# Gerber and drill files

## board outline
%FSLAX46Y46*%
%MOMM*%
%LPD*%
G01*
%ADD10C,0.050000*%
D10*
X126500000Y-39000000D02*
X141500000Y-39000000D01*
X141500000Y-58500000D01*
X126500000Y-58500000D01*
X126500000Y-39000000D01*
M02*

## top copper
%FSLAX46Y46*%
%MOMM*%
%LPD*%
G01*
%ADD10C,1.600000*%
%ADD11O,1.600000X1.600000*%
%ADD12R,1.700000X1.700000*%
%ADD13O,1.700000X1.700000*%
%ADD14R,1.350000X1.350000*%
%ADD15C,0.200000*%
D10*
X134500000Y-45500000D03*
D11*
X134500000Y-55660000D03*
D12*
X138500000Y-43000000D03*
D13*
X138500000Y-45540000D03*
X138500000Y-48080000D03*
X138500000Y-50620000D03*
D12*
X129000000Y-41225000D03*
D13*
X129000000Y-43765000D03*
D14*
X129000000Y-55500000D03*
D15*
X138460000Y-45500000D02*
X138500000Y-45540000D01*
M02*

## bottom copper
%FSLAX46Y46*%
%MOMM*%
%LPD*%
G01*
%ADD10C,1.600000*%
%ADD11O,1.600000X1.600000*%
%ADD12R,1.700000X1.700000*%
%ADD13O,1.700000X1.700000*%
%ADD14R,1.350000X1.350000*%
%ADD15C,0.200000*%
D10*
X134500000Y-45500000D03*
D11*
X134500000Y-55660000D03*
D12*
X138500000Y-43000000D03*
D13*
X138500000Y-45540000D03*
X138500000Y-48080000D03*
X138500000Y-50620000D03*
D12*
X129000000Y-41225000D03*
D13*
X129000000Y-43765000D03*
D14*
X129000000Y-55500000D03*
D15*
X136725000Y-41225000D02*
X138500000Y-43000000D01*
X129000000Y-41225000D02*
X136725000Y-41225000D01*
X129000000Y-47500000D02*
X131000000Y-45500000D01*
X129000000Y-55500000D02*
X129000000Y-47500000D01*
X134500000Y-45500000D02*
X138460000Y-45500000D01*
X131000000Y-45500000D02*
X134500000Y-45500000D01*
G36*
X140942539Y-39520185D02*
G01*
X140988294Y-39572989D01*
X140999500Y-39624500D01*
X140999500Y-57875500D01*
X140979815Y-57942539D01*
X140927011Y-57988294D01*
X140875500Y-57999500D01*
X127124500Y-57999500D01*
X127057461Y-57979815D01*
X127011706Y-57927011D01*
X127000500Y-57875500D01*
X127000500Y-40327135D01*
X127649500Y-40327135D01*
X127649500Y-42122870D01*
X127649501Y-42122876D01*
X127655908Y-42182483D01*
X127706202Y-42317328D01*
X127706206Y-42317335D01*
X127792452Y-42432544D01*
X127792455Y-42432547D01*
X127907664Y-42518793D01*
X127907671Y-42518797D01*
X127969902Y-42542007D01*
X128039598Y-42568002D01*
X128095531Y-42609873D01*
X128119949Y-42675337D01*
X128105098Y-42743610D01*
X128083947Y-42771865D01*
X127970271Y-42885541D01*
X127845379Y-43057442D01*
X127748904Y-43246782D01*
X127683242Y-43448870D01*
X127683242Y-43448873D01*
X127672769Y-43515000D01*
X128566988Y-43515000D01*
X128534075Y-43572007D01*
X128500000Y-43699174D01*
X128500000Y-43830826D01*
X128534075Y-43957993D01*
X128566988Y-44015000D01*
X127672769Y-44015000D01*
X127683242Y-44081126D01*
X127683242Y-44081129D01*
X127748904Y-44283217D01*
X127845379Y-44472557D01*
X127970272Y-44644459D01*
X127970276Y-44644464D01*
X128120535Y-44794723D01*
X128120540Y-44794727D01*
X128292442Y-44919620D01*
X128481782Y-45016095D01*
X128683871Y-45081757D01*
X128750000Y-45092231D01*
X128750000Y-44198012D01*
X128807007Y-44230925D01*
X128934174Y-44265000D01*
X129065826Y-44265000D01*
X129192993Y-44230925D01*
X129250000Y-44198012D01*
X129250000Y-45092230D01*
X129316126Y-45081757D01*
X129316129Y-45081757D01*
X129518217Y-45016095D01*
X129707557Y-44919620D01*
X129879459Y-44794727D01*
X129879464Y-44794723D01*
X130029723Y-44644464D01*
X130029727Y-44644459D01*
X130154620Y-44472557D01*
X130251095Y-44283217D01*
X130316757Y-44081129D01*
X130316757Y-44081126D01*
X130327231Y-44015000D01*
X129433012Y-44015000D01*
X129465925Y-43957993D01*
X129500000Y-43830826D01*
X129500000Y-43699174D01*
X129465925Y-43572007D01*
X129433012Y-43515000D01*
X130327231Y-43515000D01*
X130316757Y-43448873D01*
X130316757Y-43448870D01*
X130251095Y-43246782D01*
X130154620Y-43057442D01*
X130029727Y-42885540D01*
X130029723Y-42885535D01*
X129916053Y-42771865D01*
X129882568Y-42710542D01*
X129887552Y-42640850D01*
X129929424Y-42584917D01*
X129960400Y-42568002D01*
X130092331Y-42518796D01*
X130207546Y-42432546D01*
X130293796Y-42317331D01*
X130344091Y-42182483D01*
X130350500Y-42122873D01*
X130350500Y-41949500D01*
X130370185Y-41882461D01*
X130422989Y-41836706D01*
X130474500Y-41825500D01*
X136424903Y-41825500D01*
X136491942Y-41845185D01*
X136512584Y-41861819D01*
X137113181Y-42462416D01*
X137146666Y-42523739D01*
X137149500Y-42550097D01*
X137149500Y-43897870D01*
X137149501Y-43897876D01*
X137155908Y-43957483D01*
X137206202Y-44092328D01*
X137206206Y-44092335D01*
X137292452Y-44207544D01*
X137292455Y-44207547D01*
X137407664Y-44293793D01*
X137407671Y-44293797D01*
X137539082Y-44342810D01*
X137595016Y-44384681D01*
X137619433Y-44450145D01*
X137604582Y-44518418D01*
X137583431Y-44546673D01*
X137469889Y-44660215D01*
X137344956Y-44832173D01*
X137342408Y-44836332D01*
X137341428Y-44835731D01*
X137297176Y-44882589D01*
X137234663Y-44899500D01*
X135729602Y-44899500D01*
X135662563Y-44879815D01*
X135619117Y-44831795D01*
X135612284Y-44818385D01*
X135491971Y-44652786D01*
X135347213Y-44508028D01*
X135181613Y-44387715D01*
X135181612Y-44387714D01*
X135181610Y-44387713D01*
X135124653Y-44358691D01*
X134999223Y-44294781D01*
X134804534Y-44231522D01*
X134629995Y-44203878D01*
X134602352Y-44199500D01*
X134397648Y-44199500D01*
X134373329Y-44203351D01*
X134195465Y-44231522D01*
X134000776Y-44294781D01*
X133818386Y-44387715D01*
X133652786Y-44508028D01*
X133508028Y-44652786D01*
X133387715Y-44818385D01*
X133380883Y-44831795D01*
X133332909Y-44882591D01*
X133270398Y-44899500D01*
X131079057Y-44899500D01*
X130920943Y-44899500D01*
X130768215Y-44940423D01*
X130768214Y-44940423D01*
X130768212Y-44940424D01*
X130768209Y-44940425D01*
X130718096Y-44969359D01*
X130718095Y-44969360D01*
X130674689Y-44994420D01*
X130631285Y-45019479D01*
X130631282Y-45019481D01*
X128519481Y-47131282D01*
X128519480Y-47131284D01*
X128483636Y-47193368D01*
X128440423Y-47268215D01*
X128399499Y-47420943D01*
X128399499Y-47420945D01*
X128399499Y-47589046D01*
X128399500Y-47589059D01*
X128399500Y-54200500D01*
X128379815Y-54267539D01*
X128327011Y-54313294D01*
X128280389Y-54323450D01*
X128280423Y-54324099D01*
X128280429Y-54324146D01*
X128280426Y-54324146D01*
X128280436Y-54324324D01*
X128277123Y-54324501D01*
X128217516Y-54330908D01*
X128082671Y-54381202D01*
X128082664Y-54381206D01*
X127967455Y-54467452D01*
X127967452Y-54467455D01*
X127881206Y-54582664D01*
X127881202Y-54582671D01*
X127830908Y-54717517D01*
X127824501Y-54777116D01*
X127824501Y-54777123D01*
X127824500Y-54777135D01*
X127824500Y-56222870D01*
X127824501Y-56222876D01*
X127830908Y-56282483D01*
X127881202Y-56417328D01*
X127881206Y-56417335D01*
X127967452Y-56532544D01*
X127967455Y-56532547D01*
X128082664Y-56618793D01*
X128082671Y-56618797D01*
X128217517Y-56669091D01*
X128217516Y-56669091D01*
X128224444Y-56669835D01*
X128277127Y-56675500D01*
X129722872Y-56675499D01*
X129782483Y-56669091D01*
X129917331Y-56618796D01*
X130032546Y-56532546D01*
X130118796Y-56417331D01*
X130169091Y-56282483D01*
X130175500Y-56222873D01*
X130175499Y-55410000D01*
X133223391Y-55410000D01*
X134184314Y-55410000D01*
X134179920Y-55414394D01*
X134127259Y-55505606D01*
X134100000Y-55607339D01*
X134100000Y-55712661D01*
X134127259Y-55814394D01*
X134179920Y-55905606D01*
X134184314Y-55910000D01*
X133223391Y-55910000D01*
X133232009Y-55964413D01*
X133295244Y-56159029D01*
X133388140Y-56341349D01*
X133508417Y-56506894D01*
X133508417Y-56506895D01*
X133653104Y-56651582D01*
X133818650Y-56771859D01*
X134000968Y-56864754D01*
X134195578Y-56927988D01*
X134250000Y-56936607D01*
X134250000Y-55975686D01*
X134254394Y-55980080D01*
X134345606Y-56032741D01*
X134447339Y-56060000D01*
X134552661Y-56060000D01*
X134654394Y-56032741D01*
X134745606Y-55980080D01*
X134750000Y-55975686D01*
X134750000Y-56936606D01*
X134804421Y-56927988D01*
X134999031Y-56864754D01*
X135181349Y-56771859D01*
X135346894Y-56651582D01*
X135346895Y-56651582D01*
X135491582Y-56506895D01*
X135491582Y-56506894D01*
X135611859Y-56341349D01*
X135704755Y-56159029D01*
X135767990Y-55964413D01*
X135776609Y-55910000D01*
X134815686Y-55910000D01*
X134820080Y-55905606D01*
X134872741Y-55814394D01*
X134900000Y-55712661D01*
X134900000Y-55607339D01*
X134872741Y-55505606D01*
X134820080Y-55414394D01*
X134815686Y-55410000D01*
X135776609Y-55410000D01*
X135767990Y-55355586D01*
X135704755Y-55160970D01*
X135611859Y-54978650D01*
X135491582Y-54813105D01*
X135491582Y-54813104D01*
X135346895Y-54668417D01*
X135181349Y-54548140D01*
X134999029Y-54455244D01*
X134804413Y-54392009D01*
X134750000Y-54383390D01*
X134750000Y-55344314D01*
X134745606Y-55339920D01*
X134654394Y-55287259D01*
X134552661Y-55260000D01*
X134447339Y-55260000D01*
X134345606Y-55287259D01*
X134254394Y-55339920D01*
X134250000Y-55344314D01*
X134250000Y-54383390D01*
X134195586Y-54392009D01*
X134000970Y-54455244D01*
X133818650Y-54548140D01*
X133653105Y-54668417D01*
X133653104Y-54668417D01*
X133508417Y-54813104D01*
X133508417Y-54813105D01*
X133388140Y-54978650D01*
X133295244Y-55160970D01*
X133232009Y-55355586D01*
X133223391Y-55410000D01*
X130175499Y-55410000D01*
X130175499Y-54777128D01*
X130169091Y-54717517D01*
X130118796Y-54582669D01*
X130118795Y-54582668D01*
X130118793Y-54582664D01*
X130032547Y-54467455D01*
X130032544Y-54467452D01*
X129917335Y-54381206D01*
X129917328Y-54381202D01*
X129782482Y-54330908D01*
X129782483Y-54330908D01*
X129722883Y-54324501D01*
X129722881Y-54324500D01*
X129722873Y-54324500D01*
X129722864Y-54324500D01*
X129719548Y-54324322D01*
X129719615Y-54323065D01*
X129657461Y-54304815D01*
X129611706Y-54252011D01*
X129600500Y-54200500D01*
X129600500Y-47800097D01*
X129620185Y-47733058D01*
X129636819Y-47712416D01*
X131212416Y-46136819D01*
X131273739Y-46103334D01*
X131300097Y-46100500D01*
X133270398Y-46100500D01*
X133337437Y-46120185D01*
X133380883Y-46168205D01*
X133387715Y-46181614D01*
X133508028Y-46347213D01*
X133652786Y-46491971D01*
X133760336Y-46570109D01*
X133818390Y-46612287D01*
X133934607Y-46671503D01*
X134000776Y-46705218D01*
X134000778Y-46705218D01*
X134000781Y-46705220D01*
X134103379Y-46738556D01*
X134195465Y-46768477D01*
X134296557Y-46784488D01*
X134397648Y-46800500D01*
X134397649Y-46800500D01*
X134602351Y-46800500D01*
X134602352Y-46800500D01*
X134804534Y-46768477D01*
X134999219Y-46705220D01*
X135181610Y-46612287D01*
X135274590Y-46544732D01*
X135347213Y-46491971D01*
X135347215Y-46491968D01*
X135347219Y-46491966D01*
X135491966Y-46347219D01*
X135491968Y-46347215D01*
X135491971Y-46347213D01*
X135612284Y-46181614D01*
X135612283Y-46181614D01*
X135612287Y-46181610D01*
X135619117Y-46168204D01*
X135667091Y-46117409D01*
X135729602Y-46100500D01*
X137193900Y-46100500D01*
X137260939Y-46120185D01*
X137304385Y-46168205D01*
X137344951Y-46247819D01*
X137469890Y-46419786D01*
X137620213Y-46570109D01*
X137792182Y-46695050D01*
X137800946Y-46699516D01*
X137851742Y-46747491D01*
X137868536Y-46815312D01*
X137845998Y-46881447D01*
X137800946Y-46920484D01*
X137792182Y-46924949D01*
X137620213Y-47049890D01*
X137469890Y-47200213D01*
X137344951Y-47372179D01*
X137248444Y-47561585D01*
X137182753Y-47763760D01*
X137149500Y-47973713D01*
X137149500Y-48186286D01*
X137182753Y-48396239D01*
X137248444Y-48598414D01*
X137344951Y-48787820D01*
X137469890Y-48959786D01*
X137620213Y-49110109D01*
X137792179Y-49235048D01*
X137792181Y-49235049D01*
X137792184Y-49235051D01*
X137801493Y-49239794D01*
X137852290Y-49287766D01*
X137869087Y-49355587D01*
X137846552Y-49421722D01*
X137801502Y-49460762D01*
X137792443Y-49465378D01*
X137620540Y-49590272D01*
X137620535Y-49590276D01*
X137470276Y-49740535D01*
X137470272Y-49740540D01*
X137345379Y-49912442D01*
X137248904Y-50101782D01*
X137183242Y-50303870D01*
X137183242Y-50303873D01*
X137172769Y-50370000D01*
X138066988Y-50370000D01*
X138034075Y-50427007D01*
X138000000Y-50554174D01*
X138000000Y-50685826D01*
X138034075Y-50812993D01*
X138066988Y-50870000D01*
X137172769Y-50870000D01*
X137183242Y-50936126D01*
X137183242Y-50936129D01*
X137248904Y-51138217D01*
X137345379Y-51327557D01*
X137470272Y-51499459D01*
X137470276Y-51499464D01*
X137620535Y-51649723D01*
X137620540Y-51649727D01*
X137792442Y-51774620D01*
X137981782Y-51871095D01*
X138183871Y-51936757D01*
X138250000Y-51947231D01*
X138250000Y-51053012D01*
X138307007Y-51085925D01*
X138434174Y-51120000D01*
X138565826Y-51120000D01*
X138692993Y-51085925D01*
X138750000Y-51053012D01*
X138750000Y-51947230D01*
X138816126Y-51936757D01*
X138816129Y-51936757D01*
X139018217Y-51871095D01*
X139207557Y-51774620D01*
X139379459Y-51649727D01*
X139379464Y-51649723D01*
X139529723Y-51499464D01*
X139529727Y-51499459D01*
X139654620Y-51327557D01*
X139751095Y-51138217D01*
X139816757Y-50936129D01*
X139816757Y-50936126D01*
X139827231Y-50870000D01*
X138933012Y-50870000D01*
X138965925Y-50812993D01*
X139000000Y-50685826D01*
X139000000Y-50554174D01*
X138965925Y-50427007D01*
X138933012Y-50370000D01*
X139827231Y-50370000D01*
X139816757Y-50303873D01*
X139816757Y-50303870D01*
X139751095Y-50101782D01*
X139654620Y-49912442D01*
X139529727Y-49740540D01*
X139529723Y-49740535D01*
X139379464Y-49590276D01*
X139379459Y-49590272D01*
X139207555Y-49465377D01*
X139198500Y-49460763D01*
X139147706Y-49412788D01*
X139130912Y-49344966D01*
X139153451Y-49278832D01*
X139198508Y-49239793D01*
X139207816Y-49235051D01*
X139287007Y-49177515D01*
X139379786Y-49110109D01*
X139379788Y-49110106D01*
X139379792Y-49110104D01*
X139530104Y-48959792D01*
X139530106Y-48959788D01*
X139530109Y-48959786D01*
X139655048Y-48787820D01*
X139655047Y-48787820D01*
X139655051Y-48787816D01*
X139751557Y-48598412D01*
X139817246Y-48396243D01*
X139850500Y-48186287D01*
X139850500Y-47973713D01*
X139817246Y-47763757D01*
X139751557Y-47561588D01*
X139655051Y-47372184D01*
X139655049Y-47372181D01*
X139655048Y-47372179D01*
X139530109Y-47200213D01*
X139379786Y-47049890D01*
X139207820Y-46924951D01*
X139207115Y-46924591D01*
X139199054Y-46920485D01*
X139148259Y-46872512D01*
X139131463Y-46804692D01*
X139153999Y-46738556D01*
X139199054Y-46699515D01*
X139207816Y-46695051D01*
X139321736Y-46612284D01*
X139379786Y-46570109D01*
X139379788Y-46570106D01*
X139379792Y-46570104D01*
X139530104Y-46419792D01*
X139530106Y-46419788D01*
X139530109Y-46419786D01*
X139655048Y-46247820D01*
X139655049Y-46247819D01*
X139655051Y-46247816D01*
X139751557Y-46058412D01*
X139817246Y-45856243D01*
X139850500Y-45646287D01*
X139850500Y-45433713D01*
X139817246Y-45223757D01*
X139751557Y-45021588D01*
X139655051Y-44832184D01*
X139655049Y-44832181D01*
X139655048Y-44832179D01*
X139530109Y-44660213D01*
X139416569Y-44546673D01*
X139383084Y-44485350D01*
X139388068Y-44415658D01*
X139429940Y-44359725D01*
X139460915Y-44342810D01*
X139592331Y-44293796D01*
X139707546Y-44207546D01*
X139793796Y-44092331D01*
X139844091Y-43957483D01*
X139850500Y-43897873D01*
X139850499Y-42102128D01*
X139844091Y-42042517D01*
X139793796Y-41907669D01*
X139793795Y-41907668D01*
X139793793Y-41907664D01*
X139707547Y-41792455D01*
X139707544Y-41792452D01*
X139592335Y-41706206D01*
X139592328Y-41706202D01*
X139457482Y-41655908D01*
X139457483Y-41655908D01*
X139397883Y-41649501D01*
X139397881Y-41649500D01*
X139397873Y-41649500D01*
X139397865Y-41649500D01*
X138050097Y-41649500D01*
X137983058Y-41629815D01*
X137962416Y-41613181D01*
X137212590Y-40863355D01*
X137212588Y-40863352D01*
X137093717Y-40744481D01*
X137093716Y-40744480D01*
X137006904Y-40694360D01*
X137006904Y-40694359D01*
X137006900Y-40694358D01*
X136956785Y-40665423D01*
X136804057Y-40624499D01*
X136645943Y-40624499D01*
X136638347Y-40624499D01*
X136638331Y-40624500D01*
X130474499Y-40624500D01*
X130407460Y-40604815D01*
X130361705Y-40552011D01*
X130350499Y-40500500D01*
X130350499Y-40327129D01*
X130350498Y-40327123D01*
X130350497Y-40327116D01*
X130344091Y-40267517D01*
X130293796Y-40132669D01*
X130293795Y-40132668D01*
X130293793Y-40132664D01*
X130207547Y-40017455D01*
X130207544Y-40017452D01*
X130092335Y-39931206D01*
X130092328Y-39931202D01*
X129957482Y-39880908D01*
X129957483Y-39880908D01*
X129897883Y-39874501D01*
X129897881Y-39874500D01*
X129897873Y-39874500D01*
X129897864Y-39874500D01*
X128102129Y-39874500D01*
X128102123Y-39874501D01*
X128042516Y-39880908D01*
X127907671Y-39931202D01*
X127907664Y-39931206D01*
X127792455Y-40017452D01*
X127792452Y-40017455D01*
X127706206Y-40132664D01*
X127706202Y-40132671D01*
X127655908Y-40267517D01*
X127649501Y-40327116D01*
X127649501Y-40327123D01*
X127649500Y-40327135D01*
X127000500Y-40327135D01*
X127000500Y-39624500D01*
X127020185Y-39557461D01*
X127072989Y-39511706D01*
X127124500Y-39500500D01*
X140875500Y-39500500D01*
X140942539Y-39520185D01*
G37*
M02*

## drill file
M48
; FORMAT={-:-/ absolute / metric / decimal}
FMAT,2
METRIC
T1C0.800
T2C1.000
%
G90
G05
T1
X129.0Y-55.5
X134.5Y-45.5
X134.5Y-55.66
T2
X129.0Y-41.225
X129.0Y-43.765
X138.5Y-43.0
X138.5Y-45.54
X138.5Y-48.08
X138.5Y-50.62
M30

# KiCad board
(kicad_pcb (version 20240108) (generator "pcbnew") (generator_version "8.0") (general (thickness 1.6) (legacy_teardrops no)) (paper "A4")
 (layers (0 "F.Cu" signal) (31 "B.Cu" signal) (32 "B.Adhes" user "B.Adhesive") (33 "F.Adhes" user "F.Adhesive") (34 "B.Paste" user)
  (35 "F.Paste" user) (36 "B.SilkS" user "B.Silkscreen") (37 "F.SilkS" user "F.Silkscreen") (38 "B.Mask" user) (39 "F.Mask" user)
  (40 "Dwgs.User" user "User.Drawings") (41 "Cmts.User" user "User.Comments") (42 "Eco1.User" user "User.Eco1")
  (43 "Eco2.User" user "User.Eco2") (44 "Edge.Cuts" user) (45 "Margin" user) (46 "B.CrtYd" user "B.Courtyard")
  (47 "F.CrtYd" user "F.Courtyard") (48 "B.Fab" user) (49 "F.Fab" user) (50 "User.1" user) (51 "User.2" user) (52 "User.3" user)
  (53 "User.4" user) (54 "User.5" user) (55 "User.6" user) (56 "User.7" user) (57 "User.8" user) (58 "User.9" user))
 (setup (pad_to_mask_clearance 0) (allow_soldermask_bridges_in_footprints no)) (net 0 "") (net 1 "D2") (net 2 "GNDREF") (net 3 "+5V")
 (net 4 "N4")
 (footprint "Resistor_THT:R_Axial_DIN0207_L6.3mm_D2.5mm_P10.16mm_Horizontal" (layer "F.Cu") (at 134.5 45.5 -90)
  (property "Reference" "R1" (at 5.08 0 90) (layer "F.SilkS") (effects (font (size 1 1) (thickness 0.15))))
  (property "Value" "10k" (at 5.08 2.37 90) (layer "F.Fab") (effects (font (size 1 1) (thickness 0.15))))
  (pad "1" thru_hole circle (at 0 0 270) (size 1.6 1.6) (drill 0.8) (layers "*.Cu" "*.Mask") (remove_unused_layers no) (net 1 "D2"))
  (pad "2" thru_hole oval (at 10.16 0 270) (size 1.6 1.6) (drill 0.8) (layers "*.Cu" "*.Mask") (remove_unused_layers no) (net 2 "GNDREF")))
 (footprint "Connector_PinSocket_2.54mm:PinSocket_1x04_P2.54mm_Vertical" (layer "F.Cu") (at 138.5 43)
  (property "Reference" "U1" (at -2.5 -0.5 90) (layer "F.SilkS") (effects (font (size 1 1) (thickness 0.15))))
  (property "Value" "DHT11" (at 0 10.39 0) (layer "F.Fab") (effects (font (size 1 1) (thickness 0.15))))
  (pad "1" thru_hole rect (at 0 0) (size 1.7 1.7) (drill 1) (layers "*.Cu" "*.Mask") (remove_unused_layers no) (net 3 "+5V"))
  (pad "2" thru_hole oval (at 0 2.54) (size 1.7 1.7) (drill 1) (layers "*.Cu" "*.Mask") (remove_unused_layers no) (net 1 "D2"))
  (pad "3" thru_hole oval (at 0 5.08) (size 1.7 1.7) (drill 1) (layers "*.Cu" "*.Mask") (remove_unused_layers no) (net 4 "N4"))
  (pad "4" thru_hole oval (at 0 7.62) (size 1.7 1.7) (drill 1) (layers "*.Cu" "*.Mask") (remove_unused_layers no) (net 2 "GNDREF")))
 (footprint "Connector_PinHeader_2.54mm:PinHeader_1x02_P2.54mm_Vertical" (layer "F.Cu") (at 129 41.225)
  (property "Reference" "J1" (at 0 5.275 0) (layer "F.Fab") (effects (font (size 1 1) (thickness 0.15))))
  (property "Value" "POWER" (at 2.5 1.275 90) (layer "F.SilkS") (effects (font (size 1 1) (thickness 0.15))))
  (pad "1" thru_hole rect (at 0 0) (size 1.7 1.7) (drill 1) (layers "*.Cu" "*.Mask") (remove_unused_layers no) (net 3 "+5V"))
  (pad "2" thru_hole oval (at 0 2.54) (size 1.7 1.7) (drill 1) (layers "*.Cu" "*.Mask") (remove_unused_layers no) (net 2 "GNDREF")))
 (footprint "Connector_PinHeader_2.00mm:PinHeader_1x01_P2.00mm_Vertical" (layer "F.Cu") (at 129 55.5)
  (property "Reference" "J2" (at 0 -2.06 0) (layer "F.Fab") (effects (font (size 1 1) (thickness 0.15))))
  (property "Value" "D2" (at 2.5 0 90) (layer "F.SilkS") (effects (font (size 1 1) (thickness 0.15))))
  (pad "1" thru_hole rect (at 0 0) (size 1.35 1.35) (drill 0.8) (layers "*.Cu" "*.Mask") (remove_unused_layers no) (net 1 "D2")))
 (gr_rect (start 126.5 39) (end 141.5 58.5) (stroke (width 0.05) (type default)) (fill none) (layer "Edge.Cuts"))
 (segment (start 136.725 41.225) (end 138.5 43) (width 0.2) (layer "B.Cu") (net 3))
 (segment (start 129 41.225) (end 136.725 41.225) (width 0.2) (layer "B.Cu") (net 3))
 (segment (start 138.46 45.5) (end 138.5 45.54) (width 0.2) (layer "F.Cu") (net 1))
 (segment (start 129 47.5) (end 131 45.5) (width 0.2) (layer "B.Cu") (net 1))
 (segment (start 129 55.5) (end 129 47.5) (width 0.2) (layer "B.Cu") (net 1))
 (segment (start 134.5 45.5) (end 138.46 45.5) (width 0.2) (layer "B.Cu") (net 1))
 (segment (start 131 45.5) (end 134.5 45.5) (width 0.2) (layer "B.Cu") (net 1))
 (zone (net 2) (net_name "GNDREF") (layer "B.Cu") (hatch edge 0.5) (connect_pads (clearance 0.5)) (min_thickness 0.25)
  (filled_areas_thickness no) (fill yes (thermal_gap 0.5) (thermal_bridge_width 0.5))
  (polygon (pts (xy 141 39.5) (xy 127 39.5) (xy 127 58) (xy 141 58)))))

